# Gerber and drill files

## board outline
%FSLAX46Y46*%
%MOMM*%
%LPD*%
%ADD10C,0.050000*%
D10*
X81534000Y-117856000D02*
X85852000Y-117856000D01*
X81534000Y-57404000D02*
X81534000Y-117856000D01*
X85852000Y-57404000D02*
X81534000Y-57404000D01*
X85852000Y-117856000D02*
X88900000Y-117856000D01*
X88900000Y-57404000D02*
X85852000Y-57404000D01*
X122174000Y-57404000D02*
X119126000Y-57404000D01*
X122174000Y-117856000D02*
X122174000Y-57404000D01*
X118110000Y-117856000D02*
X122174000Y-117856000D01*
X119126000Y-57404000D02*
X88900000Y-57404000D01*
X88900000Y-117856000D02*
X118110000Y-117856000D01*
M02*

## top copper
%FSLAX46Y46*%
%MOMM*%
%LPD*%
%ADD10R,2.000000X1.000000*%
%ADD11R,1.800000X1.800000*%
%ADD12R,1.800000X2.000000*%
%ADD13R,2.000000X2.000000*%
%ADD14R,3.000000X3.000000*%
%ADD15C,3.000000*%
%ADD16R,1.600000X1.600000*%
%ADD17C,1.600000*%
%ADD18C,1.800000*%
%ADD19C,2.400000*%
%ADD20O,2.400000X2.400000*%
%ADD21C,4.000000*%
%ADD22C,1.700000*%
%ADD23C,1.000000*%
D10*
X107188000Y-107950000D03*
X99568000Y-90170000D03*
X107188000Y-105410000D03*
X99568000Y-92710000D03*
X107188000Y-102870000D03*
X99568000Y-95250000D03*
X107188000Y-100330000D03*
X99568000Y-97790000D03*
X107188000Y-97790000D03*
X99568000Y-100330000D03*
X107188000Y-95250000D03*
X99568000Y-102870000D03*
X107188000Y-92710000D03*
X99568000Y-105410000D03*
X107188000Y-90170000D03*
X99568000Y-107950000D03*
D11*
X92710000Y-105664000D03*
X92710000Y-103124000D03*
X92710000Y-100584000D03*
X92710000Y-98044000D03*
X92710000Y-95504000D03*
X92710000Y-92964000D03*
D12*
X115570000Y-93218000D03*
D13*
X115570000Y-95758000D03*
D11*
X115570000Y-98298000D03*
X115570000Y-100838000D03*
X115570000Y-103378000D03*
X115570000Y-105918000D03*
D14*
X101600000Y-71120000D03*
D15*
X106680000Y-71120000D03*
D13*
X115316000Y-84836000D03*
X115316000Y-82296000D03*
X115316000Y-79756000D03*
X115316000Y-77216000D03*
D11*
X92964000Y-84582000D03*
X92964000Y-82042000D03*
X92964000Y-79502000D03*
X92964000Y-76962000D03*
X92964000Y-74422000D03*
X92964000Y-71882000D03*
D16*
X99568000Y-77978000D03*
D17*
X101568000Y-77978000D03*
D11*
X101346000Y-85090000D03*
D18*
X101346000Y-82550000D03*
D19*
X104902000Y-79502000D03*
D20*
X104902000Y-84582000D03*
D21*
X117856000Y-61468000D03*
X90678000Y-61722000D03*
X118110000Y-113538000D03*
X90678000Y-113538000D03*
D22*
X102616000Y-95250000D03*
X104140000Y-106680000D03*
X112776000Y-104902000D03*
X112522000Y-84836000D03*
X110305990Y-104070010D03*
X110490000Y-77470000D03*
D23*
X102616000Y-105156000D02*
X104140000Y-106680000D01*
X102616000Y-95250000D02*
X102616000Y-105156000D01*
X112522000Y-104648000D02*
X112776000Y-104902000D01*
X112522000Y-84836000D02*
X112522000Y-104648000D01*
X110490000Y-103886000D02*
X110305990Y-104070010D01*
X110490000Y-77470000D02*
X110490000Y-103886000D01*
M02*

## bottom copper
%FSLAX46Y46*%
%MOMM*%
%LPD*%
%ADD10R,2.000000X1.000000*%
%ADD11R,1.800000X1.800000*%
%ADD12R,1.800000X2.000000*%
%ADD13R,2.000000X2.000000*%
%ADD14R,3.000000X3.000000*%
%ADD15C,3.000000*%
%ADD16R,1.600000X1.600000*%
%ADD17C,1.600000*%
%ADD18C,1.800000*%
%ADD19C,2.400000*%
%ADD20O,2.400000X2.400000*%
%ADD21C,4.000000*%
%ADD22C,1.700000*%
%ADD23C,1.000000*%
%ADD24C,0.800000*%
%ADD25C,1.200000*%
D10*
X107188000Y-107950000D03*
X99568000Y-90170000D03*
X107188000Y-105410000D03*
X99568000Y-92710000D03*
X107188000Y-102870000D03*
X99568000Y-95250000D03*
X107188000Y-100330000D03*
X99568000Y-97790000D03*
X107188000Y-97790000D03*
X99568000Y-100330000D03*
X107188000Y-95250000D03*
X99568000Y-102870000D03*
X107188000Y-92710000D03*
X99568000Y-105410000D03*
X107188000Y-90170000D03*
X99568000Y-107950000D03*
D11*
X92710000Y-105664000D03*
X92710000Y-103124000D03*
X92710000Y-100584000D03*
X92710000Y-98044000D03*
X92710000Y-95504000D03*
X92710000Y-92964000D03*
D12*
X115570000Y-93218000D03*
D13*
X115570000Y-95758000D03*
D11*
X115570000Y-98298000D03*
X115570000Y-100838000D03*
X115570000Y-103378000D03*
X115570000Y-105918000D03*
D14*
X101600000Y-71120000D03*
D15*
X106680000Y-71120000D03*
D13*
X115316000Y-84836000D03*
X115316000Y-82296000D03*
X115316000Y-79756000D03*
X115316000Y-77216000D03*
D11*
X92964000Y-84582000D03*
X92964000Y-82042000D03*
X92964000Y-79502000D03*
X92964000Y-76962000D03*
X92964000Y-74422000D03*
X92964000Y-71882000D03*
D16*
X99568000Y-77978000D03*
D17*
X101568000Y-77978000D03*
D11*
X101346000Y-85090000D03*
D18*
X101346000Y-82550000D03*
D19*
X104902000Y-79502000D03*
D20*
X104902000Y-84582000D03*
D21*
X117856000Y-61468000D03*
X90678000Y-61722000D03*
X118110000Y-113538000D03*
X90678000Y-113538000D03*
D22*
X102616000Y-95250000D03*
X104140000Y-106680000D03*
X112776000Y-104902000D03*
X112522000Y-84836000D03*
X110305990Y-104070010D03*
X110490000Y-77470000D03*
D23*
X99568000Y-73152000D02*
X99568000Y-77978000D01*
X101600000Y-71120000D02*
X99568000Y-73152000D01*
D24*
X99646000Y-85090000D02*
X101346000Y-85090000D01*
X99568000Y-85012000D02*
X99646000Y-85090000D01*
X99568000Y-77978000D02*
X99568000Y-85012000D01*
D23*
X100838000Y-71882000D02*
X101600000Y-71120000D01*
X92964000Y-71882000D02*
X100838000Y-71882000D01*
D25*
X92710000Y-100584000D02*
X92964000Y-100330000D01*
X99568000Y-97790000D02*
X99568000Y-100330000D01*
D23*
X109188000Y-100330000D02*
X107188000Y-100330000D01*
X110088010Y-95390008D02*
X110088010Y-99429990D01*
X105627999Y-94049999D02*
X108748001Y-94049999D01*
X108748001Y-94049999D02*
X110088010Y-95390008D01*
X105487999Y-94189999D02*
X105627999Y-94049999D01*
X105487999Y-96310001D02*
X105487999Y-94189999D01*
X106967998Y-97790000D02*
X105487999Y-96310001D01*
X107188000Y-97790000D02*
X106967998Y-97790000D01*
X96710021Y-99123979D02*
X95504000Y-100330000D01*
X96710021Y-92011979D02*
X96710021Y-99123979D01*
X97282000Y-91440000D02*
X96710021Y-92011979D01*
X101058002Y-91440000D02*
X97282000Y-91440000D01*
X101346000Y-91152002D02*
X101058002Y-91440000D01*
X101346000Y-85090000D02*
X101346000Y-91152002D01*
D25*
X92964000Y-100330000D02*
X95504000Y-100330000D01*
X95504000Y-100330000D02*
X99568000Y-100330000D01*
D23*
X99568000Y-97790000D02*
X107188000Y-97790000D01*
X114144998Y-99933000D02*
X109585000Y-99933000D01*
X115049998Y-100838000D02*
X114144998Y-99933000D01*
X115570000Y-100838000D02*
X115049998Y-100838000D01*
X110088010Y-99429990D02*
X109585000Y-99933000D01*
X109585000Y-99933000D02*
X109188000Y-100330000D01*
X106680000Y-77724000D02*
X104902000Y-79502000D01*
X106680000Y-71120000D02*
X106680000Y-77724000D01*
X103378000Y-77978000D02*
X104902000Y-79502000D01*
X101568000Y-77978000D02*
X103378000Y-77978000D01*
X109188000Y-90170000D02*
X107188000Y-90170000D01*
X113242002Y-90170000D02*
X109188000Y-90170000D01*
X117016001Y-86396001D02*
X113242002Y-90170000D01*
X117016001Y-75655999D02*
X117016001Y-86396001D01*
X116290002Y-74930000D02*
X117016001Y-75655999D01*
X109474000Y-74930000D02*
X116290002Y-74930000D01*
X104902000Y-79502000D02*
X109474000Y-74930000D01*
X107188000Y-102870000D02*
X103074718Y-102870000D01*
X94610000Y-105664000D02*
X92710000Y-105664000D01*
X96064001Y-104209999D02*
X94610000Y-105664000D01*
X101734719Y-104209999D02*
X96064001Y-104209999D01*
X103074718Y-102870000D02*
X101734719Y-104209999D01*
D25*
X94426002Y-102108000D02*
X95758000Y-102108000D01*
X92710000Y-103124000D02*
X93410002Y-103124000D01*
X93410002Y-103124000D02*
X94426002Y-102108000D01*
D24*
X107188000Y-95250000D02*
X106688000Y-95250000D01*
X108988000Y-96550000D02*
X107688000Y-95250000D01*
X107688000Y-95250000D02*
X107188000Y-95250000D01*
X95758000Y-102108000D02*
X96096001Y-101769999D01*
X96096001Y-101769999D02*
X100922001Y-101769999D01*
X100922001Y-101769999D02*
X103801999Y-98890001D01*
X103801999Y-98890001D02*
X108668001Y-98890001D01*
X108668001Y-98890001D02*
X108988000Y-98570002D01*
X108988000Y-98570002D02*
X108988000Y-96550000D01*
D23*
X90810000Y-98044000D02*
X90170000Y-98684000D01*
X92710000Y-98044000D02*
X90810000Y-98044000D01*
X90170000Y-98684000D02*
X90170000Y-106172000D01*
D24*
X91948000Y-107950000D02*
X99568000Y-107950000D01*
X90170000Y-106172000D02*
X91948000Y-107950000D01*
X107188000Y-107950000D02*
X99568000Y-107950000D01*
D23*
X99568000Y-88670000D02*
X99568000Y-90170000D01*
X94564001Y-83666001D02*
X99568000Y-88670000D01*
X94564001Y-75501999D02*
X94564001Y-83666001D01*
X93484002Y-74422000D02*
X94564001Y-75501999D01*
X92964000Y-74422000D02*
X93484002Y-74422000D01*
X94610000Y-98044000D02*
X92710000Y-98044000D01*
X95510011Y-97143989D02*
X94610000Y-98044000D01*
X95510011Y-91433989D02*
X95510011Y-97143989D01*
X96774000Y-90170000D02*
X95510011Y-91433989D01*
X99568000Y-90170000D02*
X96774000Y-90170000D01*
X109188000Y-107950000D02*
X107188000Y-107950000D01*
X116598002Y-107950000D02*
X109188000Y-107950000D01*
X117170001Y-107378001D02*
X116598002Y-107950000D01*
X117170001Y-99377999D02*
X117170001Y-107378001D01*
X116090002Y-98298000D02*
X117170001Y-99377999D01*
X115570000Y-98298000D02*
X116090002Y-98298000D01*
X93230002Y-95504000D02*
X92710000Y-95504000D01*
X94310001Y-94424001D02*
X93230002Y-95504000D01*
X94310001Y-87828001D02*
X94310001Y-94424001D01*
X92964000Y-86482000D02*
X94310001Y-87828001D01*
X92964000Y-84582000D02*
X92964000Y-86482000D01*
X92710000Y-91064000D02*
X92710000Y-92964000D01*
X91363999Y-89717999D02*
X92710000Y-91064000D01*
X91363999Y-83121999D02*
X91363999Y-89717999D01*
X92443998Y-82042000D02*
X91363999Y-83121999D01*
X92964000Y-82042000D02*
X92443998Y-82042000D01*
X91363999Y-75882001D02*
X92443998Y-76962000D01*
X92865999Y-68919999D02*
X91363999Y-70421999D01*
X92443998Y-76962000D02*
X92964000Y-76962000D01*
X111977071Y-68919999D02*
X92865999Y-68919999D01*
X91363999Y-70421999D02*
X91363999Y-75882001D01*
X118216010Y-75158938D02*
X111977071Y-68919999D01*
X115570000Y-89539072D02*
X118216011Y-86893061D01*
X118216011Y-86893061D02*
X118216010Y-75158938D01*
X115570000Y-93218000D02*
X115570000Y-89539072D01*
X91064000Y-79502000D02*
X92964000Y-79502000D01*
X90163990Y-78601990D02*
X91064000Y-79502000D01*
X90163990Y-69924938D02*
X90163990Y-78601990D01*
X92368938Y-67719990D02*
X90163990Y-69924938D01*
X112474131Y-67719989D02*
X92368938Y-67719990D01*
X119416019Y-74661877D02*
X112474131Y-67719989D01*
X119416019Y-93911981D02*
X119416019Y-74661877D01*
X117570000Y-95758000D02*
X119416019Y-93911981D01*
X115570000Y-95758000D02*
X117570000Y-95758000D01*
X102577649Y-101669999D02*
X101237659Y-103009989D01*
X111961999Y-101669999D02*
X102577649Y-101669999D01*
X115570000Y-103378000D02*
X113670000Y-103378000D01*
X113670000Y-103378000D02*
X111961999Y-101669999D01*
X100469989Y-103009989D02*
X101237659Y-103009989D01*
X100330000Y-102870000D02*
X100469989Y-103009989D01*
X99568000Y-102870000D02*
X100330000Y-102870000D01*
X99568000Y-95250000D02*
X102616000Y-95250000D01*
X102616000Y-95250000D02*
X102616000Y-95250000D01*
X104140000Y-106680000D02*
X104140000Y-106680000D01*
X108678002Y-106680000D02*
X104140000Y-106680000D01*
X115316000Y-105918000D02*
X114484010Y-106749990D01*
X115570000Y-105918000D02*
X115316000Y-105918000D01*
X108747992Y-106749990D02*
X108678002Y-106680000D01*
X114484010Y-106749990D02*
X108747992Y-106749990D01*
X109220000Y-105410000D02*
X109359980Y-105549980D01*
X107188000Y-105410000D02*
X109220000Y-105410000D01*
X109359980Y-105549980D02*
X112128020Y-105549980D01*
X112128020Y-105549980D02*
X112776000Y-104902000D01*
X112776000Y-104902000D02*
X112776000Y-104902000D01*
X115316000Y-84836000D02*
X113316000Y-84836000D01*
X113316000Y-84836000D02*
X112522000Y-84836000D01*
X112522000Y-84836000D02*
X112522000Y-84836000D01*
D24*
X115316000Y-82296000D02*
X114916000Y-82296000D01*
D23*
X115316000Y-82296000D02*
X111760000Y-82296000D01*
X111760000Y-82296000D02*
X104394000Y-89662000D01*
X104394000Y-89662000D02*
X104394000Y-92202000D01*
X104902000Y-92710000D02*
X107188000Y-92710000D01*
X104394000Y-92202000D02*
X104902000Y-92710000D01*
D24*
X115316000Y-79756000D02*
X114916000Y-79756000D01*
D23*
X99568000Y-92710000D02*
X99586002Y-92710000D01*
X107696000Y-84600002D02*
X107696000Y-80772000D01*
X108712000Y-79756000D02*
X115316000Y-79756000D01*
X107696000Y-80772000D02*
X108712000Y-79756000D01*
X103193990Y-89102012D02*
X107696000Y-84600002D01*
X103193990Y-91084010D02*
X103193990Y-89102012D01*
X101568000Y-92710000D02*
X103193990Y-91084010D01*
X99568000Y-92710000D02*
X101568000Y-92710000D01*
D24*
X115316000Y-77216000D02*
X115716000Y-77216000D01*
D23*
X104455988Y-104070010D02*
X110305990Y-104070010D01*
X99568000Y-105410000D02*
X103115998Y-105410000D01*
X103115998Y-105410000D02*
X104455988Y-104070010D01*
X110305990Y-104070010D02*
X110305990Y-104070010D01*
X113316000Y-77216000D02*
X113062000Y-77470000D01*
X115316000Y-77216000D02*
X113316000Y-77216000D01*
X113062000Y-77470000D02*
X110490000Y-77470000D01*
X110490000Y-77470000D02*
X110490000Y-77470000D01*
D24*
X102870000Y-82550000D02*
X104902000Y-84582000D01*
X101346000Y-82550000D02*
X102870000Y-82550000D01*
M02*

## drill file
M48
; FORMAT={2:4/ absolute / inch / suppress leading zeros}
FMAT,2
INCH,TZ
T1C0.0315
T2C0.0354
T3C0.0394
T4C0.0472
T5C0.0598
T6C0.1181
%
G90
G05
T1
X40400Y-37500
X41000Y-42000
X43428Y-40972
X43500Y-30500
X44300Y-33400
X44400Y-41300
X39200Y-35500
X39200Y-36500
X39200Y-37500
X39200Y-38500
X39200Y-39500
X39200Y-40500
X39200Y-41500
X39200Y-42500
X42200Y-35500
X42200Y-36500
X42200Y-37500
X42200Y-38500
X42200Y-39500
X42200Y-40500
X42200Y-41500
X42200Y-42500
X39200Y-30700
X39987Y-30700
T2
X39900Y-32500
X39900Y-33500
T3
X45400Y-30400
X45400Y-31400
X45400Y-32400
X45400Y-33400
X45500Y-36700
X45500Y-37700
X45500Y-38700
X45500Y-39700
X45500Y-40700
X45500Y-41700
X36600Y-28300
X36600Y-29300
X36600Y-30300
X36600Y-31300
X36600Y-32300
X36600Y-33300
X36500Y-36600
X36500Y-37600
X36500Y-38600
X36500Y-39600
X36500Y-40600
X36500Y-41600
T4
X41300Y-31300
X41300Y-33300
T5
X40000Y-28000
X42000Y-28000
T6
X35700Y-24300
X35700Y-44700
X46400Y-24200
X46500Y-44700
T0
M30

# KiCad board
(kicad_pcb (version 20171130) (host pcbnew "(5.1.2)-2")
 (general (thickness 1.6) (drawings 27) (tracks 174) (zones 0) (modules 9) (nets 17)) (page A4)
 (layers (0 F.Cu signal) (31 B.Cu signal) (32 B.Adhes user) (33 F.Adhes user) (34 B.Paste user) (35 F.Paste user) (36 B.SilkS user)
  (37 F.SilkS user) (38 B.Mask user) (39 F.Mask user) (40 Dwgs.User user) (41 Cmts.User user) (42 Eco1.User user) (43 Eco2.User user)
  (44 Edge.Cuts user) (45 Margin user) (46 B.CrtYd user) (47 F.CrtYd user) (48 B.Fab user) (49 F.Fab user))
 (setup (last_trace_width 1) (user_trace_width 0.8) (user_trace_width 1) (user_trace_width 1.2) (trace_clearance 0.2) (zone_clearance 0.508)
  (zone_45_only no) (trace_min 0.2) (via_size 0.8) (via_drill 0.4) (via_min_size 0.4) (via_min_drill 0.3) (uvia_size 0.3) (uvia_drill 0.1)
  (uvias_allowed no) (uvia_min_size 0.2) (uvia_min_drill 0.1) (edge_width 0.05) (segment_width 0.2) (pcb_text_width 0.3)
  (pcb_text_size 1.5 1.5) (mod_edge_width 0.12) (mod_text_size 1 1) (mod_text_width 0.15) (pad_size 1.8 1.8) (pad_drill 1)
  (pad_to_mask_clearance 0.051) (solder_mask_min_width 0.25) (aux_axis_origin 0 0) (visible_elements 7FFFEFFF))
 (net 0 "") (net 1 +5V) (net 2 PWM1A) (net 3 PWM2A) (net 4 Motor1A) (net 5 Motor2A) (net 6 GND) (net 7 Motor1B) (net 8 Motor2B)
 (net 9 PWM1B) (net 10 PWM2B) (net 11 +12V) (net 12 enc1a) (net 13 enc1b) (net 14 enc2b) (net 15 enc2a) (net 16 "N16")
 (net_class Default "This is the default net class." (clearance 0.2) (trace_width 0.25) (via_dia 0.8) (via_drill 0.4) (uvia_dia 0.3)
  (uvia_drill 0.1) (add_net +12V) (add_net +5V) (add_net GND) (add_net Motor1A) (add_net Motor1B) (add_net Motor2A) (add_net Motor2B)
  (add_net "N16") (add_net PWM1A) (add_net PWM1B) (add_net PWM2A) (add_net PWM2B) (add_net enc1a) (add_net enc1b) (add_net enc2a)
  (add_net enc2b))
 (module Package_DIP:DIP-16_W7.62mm (layer F.Cu) (at 107.188 107.95 180)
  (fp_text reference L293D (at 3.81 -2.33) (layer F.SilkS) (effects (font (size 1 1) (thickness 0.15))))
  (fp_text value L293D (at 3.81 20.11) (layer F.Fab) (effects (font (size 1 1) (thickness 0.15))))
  (pad 1 thru_hole rect (at 0 0 180) (size 2 1) (drill 0.8) (layers *.Cu *.Mask) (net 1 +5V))
  (pad 9 thru_hole rect (at 7.62 17.78 180) (size 2 1) (drill 0.8) (layers *.Cu *.Mask) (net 1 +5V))
  (pad 2 thru_hole rect (at 0 2.54 180) (size 2 1) (drill 0.8) (layers *.Cu *.Mask) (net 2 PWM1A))
  (pad 10 thru_hole rect (at 7.62 15.24 180) (size 2 1) (drill 0.8) (layers *.Cu *.Mask) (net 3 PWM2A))
  (pad 3 thru_hole rect (at 0 5.08 180) (size 2 1) (drill 0.8) (layers *.Cu *.Mask) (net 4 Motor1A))
  (pad 11 thru_hole rect (at 7.62 12.7 180) (size 2 1) (drill 0.8) (layers *.Cu *.Mask) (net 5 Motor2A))
  (pad 4 thru_hole rect (at 0 7.62 180) (size 2 1) (drill 0.8) (layers *.Cu *.Mask) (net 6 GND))
  (pad 12 thru_hole rect (at 7.62 10.16 180) (size 2 1) (drill 0.8) (layers *.Cu *.Mask) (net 6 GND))
  (pad 5 thru_hole rect (at 0 10.16 180) (size 2 1) (drill 0.8) (layers *.Cu *.Mask) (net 6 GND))
  (pad 13 thru_hole rect (at 7.62 7.62 180) (size 2 1) (drill 0.8) (layers *.Cu *.Mask) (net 6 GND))
  (pad 6 thru_hole rect (at 0 12.7 180) (size 2 1) (drill 0.8) (layers *.Cu *.Mask) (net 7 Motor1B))
  (pad 14 thru_hole rect (at 7.62 5.08 180) (size 2 1) (drill 0.8) (layers *.Cu *.Mask) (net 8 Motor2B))
  (pad 7 thru_hole rect (at 0 15.24 180) (size 2 1) (drill 0.8) (layers *.Cu *.Mask) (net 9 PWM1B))
  (pad 15 thru_hole rect (at 7.62 2.54 180) (size 2 1) (drill 0.8) (layers *.Cu *.Mask) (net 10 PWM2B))
  (pad 8 thru_hole rect (at 0 17.78 180) (size 2 1) (drill 0.8) (layers *.Cu *.Mask) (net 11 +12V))
  (pad 16 thru_hole rect (at 7.62 0 180) (size 2 1) (drill 0.8) (layers *.Cu *.Mask) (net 1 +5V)))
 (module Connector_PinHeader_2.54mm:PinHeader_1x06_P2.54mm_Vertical (layer F.Cu) (at 92.71 105.664 180)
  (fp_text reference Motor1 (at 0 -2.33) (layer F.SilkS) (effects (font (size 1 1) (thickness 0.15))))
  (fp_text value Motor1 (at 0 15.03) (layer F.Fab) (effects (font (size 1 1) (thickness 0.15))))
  (pad 1 thru_hole rect (at 0 0 180) (size 1.8 1.8) (drill 1) (layers *.Cu *.Mask) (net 4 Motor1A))
  (pad 2 thru_hole rect (at 0 2.54 180) (size 1.8 1.8) (drill 1) (layers *.Cu *.Mask) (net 7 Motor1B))
  (pad 3 thru_hole rect (at 0 5.08 180) (size 1.8 1.8) (drill 1) (layers *.Cu *.Mask) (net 6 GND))
  (pad 4 thru_hole rect (at 0 7.62 180) (size 1.8 1.8) (drill 1) (layers *.Cu *.Mask) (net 1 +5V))
  (pad 5 thru_hole rect (at 0 10.16 180) (size 1.8 1.8) (drill 1) (layers *.Cu *.Mask) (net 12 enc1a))
  (pad 6 thru_hole rect (at 0 12.7 180) (size 1.8 1.8) (drill 1) (layers *.Cu *.Mask) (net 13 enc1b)))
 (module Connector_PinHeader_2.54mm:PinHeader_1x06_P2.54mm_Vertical (layer F.Cu) (at 115.57 105.918 180)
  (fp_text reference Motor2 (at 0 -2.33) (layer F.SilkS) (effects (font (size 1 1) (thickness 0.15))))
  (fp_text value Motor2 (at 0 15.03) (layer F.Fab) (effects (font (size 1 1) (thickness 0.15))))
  (pad 6 thru_hole rect (at 0 12.7 180) (size 1.8 2) (drill 1) (layers *.Cu *.Mask) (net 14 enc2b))
  (pad 5 thru_hole rect (at 0 10.16 180) (size 2 2) (drill 1) (layers *.Cu *.Mask) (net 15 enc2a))
  (pad 4 thru_hole rect (at 0 7.62 180) (size 1.8 1.8) (drill 1) (layers *.Cu *.Mask) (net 1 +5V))
  (pad 3 thru_hole rect (at 0 5.08 180) (size 1.8 1.8) (drill 1) (layers *.Cu *.Mask) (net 6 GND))
  (pad 2 thru_hole rect (at 0 2.54 180) (size 1.8 1.8) (drill 1) (layers *.Cu *.Mask) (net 8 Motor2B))
  (pad 1 thru_hole rect (at 0 0 180) (size 1.8 1.8) (drill 1) (layers *.Cu *.Mask) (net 5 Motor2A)))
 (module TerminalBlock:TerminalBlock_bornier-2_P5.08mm (layer F.Cu) (at 101.6 71.12)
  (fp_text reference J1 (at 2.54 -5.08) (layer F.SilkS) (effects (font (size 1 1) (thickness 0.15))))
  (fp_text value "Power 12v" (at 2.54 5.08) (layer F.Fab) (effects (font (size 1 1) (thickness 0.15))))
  (pad 1 thru_hole rect (at 0 0) (size 3 3) (drill 1.52) (layers *.Cu *.Mask) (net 6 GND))
  (pad 2 thru_hole circle (at 5.08 0) (size 3 3) (drill 1.52) (layers *.Cu *.Mask) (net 11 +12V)))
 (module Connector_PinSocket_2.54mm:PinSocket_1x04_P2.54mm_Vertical (layer F.Cu) (at 115.316 84.836 180)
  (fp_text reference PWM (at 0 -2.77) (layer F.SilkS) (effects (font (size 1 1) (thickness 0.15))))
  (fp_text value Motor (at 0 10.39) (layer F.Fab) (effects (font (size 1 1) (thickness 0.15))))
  (pad 1 thru_hole rect (at 0 0 180) (size 2 2) (drill 1) (layers *.Cu *.Mask) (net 2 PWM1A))
  (pad 2 thru_hole rect (at 0 2.54 180) (size 2 2) (drill 1) (layers *.Cu *.Mask) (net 9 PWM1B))
  (pad 3 thru_hole rect (at 0 5.08 180) (size 2 2) (drill 1) (layers *.Cu *.Mask) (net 3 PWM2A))
  (pad 4 thru_hole rect (at 0 7.62 180) (size 2 2) (drill 1) (layers *.Cu *.Mask) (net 10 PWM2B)))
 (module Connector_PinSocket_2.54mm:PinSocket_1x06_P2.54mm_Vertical (layer F.Cu) (at 92.964 84.582 180)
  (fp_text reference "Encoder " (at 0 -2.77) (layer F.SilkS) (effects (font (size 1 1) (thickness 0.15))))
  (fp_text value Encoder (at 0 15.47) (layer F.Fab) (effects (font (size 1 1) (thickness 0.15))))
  (pad 1 thru_hole rect (at 0 0 180) (size 1.8 1.8) (drill 1) (layers *.Cu *.Mask) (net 12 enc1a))
  (pad 2 thru_hole rect (at 0 2.54 180) (size 1.8 1.8) (drill 1) (layers *.Cu *.Mask) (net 13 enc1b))
  (pad 3 thru_hole rect (at 0 5.08 180) (size 1.8 1.8) (drill 1) (layers *.Cu *.Mask) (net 15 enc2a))
  (pad 4 thru_hole rect (at 0 7.62 180) (size 1.8 1.8) (drill 1) (layers *.Cu *.Mask) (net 14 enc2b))
  (pad 5 thru_hole rect (at 0 10.16 180) (size 1.8 1.8) (drill 1) (layers *.Cu *.Mask) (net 1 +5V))
  (pad 6 thru_hole rect (at 0 12.7 180) (size 1.8 1.8) (drill 1) (layers *.Cu *.Mask) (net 6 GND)))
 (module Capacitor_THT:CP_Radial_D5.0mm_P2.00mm (layer F.Cu) (at 99.568 77.978)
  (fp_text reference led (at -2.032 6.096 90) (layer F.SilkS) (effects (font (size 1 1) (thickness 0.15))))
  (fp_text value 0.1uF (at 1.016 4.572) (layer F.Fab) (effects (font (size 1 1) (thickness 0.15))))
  (pad 1 thru_hole rect (at 0 0) (size 1.6 1.6) (drill 0.8) (layers *.Cu *.Mask) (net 6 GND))
  (pad 2 thru_hole circle (at 2 0) (size 1.6 1.6) (drill 0.8) (layers *.Cu *.Mask) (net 11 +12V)))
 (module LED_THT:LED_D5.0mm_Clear (layer F.Cu) (at 101.346 85.09 90)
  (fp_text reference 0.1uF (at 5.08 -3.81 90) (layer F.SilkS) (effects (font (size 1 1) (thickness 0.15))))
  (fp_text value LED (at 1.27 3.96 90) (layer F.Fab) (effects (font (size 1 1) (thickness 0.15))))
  (pad 1 thru_hole rect (at 0 0 90) (size 1.8 1.8) (drill 0.9) (layers *.Cu *.Mask) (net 6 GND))
  (pad 2 thru_hole circle (at 2.54 0 90) (size 1.8 1.8) (drill 0.9) (layers *.Cu *.Mask) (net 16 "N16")))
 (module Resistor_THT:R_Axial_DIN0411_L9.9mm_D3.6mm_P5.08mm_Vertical (layer F.Cu) (at 104.902 79.502 270)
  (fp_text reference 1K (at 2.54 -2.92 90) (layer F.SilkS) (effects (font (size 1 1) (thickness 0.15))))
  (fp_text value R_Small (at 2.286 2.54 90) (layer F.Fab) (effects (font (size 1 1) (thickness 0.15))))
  (pad 1 thru_hole circle (at 0 0 270) (size 2.4 2.4) (drill 1.2) (layers *.Cu *.Mask) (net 11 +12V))
  (pad 2 thru_hole oval (at 5.08 0 270) (size 2.4 2.4) (drill 1.2) (layers *.Cu *.Mask) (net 16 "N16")))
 (gr_line (start 81.534 117.856) (end 85.852 117.856) (layer Edge.Cuts) (width 0.05))
 (gr_line (start 81.534 57.404) (end 81.534 117.856) (layer Edge.Cuts) (width 0.05))
 (gr_line (start 85.852 57.404) (end 81.534 57.404) (layer Edge.Cuts) (width 0.05))
 (gr_line (start 85.852 117.856) (end 88.9 117.856) (layer Edge.Cuts) (width 0.05))
 (gr_line (start 88.9 57.404) (end 85.852 57.404) (layer Edge.Cuts) (width 0.05))
 (gr_line (start 122.174 57.404) (end 119.126 57.404) (layer Edge.Cuts) (width 0.05))
 (gr_line (start 122.174 117.856) (end 122.174 57.404) (layer Edge.Cuts) (width 0.05))
 (gr_line (start 118.11 117.856) (end 122.174 117.856) (layer Edge.Cuts) (width 0.05))
 (gr_line (start 119.126 57.404) (end 88.9 57.404) (layer Edge.Cuts) (width 0.05))
 (gr_line (start 88.9 117.856) (end 118.11 117.856) (layer Edge.Cuts) (width 0.05))
 (via (at 117.856 61.468) (size 4) (drill 3) (layers F.Cu B.Cu) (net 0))
 (via (at 90.678 61.722) (size 4) (drill 3) (layers F.Cu B.Cu) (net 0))
 (via (at 118.11 113.538) (size 4) (drill 3) (layers F.Cu B.Cu) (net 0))
 (via (at 90.678 113.538) (size 4) (drill 3) (layers F.Cu B.Cu) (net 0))
 (segment (start 99.568 73.152) (end 99.568 77.978) (width 1) (layer B.Cu) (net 6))
 (segment (start 101.6 71.12) (end 99.568 73.152) (width 1) (layer B.Cu) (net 6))
 (segment (start 99.646 85.09) (end 101.346 85.09) (width 0.8) (layer B.Cu) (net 6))
 (segment (start 99.568 85.012) (end 99.646 85.09) (width 0.8) (layer B.Cu) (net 6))
 (segment (start 99.568 77.978) (end 99.568 85.012) (width 0.8) (layer B.Cu) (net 6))
 (segment (start 100.838 71.882) (end 101.6 71.12) (width 1) (layer B.Cu) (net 6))
 (segment (start 92.964 71.882) (end 100.838 71.882) (width 1) (layer B.Cu) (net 6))
 (segment (start 92.71 100.584) (end 92.964 100.33) (width 1.2) (layer B.Cu) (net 6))
 (segment (start 99.568 97.79) (end 99.568 100.33) (width 1.2) (layer B.Cu) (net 6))
 (segment (start 109.188 100.33) (end 107.188 100.33) (width 1) (layer B.Cu) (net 6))
 (segment (start 110.08801 95.390008) (end 110.08801 99.42999) (width 1) (layer B.Cu) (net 6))
 (segment (start 105.627999 94.049999) (end 108.748001 94.049999) (width 1) (layer B.Cu) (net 6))
 (segment (start 108.748001 94.049999) (end 110.08801 95.390008) (width 1) (layer B.Cu) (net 6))
 (segment (start 105.487999 94.189999) (end 105.627999 94.049999) (width 1) (layer B.Cu) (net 6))
 (segment (start 105.487999 96.310001) (end 105.487999 94.189999) (width 1) (layer B.Cu) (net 6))
 (segment (start 106.967998 97.79) (end 105.487999 96.310001) (width 1) (layer B.Cu) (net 6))
 (segment (start 107.188 97.79) (end 106.967998 97.79) (width 1) (layer B.Cu) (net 6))
 (segment (start 96.710021 99.123979) (end 95.504 100.33) (width 1) (layer B.Cu) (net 6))
 (segment (start 96.710021 92.011979) (end 96.710021 99.123979) (width 1) (layer B.Cu) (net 6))
 (segment (start 97.282 91.44) (end 96.710021 92.011979) (width 1) (layer B.Cu) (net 6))
 (segment (start 101.058002 91.44) (end 97.282 91.44) (width 1) (layer B.Cu) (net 6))
 (segment (start 101.346 91.152002) (end 101.058002 91.44) (width 1) (layer B.Cu) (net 6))
 (segment (start 101.346 85.09) (end 101.346 91.152002) (width 1) (layer B.Cu) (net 6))
 (segment (start 92.964 100.33) (end 95.504 100.33) (width 1.2) (layer B.Cu) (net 6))
 (segment (start 95.504 100.33) (end 99.568 100.33) (width 1.2) (layer B.Cu) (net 6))
 (segment (start 99.568 97.79) (end 107.188 97.79) (width 1) (layer B.Cu) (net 6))
 (segment (start 114.144998 99.933) (end 109.585 99.933) (width 1) (layer B.Cu) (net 6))
 (segment (start 115.049998 100.838) (end 114.144998 99.933) (width 1) (layer B.Cu) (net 6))
 (segment (start 115.57 100.838) (end 115.049998 100.838) (width 1) (layer B.Cu) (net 6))
 (segment (start 110.08801 99.42999) (end 109.585 99.933) (width 1) (layer B.Cu) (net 6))
 (segment (start 109.585 99.933) (end 109.188 100.33) (width 1) (layer B.Cu) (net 6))
 (segment (start 106.68 77.724) (end 104.902 79.502) (width 1) (layer B.Cu) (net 11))
 (segment (start 106.68 71.12) (end 106.68 77.724) (width 1) (layer B.Cu) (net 11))
 (segment (start 103.378 77.978) (end 104.902 79.502) (width 1) (layer B.Cu) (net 11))
 (segment (start 101.568 77.978) (end 103.378 77.978) (width 1) (layer B.Cu) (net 11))
 (segment (start 109.188 90.17) (end 107.188 90.17) (width 1) (layer B.Cu) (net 11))
 (segment (start 113.242002 90.17) (end 109.188 90.17) (width 1) (layer B.Cu) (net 11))
 (segment (start 117.016001 86.396001) (end 113.242002 90.17) (width 1) (layer B.Cu) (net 11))
 (segment (start 117.016001 75.655999) (end 117.016001 86.396001) (width 1) (layer B.Cu) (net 11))
 (segment (start 116.290002 74.93) (end 117.016001 75.655999) (width 1) (layer B.Cu) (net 11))
 (segment (start 109.474 74.93) (end 116.290002 74.93) (width 1) (layer B.Cu) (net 11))
 (segment (start 104.902 79.502) (end 109.474 74.93) (width 1) (layer B.Cu) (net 11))
 (segment (start 107.188 102.87) (end 103.074718 102.87) (width 1) (layer B.Cu) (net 4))
 (segment (start 94.61 105.664) (end 92.71 105.664) (width 1) (layer B.Cu) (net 4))
 (segment (start 96.064001 104.209999) (end 94.61 105.664) (width 1) (layer B.Cu) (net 4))
 (segment (start 101.734719 104.209999) (end 96.064001 104.209999) (width 1) (layer B.Cu) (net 4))
 (segment (start 103.074718 102.87) (end 101.734719 104.209999) (width 1) (layer B.Cu) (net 4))
 (segment (start 94.426002 102.108) (end 95.758 102.108) (width 1.2) (layer B.Cu) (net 7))
 (segment (start 92.71 103.124) (end 93.410002 103.124) (width 1.2) (layer B.Cu) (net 7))
 (segment (start 93.410002 103.124) (end 94.426002 102.108) (width 1.2) (layer B.Cu) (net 7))
 (segment (start 107.188 95.25) (end 106.688 95.25) (width 0.8) (layer B.Cu) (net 7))
 (segment (start 108.988 96.55) (end 107.688 95.25) (width 0.8) (layer B.Cu) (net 7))
 (segment (start 107.688 95.25) (end 107.188 95.25) (width 0.8) (layer B.Cu) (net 7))
 (segment (start 95.758 102.108) (end 96.096001 101.769999) (width 0.8) (layer B.Cu) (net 7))
 (segment (start 96.096001 101.769999) (end 100.922001 101.769999) (width 0.8) (layer B.Cu) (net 7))
 (segment (start 100.922001 101.769999) (end 103.801999 98.890001) (width 0.8) (layer B.Cu) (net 7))
 (segment (start 103.801999 98.890001) (end 108.668001 98.890001) (width 0.8) (layer B.Cu) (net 7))
 (segment (start 108.668001 98.890001) (end 108.988 98.570002) (width 0.8) (layer B.Cu) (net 7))
 (segment (start 108.988 98.570002) (end 108.988 96.55) (width 0.8) (layer B.Cu) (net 7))
 (segment (start 90.81 98.044) (end 90.17 98.684) (width 1) (layer B.Cu) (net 1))
 (segment (start 92.71 98.044) (end 90.81 98.044) (width 1) (layer B.Cu) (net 1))
 (segment (start 90.17 98.684) (end 90.17 106.172) (width 1) (layer B.Cu) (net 1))
 (segment (start 91.948 107.95) (end 99.568 107.95) (width 0.8) (layer B.Cu) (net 1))
 (segment (start 90.17 106.172) (end 91.948 107.95) (width 0.8) (layer B.Cu) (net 1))
 (segment (start 107.188 107.95) (end 99.568 107.95) (width 0.8) (layer B.Cu) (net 1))
 (segment (start 99.568 88.67) (end 99.568 90.17) (width 1) (layer B.Cu) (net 1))
 (segment (start 94.564001 83.666001) (end 99.568 88.67) (width 1) (layer B.Cu) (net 1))
 (segment (start 94.564001 75.501999) (end 94.564001 83.666001) (width 1) (layer B.Cu) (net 1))
 (segment (start 93.484002 74.422) (end 94.564001 75.501999) (width 1) (layer B.Cu) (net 1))
 (segment (start 92.964 74.422) (end 93.484002 74.422) (width 1) (layer B.Cu) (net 1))
 (segment (start 94.61 98.044) (end 92.71 98.044) (width 1) (layer B.Cu) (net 1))
 (segment (start 95.510011 97.143989) (end 94.61 98.044) (width 1) (layer B.Cu) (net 1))
 (segment (start 95.510011 91.433989) (end 95.510011 97.143989) (width 1) (layer B.Cu) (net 1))
 (segment (start 96.774 90.17) (end 95.510011 91.433989) (width 1) (layer B.Cu) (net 1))
 (segment (start 99.568 90.17) (end 96.774 90.17) (width 1) (layer B.Cu) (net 1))
 (segment (start 109.188 107.95) (end 107.188 107.95) (width 1) (layer B.Cu) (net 1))
 (segment (start 116.598002 107.95) (end 109.188 107.95) (width 1) (layer B.Cu) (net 1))
 (segment (start 117.170001 107.378001) (end 116.598002 107.95) (width 1) (layer B.Cu) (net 1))
 (segment (start 117.170001 99.377999) (end 117.170001 107.378001) (width 1) (layer B.Cu) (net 1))
 (segment (start 116.090002 98.298) (end 117.170001 99.377999) (width 1) (layer B.Cu) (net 1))
 (segment (start 115.57 98.298) (end 116.090002 98.298) (width 1) (layer B.Cu) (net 1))
 (segment (start 93.230002 95.504) (end 92.71 95.504) (width 1) (layer B.Cu) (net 12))
 (segment (start 94.310001 94.424001) (end 93.230002 95.504) (width 1) (layer B.Cu) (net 12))
 (segment (start 94.310001 87.828001) (end 94.310001 94.424001) (width 1) (layer B.Cu) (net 12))
 (segment (start 92.964 86.482) (end 94.310001 87.828001) (width 1) (layer B.Cu) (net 12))
 (segment (start 92.964 84.582) (end 92.964 86.482) (width 1) (layer B.Cu) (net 12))
 (segment (start 92.71 91.064) (end 92.71 92.964) (width 1) (layer B.Cu) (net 13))
 (segment (start 91.363999 89.717999) (end 92.71 91.064) (width 1) (layer B.Cu) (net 13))
 (segment (start 91.363999 83.121999) (end 91.363999 89.717999) (width 1) (layer B.Cu) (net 13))
 (segment (start 92.443998 82.042) (end 91.363999 83.121999) (width 1) (layer B.Cu) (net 13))
 (segment (start 92.964 82.042) (end 92.443998 82.042) (width 1) (layer B.Cu) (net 13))
 (segment (start 91.363999 75.882001) (end 92.443998 76.962) (width 1) (layer B.Cu) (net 14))
 (segment (start 92.865999 68.919999) (end 91.363999 70.421999) (width 1) (layer B.Cu) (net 14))
 (segment (start 92.443998 76.962) (end 92.964 76.962) (width 1) (layer B.Cu) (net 14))
 (segment (start 111.977071 68.919999) (end 92.865999 68.919999) (width 1) (layer B.Cu) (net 14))
 (segment (start 91.363999 70.421999) (end 91.363999 75.882001) (width 1) (layer B.Cu) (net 14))
 (segment (start 118.21601 75.158938) (end 111.977071 68.919999) (width 1) (layer B.Cu) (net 14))
 (segment (start 115.57 89.539072) (end 118.216011 86.893061) (width 1) (layer B.Cu) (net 14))
 (segment (start 118.216011 86.893061) (end 118.21601 75.158938) (width 1) (layer B.Cu) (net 14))
 (segment (start 115.57 93.218) (end 115.57 89.539072) (width 1) (layer B.Cu) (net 14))
 (segment (start 91.064 79.502) (end 92.964 79.502) (width 1) (layer B.Cu) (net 15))
 (segment (start 90.16399 78.60199) (end 91.064 79.502) (width 1) (layer B.Cu) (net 15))
 (segment (start 90.16399 69.924938) (end 90.16399 78.60199) (width 1) (layer B.Cu) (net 15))
 (segment (start 92.368938 67.71999) (end 90.16399 69.924938) (width 1) (layer B.Cu) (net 15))
 (segment (start 112.474131 67.719989) (end 92.368938 67.71999) (width 1) (layer B.Cu) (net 15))
 (segment (start 119.416019 74.661877) (end 112.474131 67.719989) (width 1) (layer B.Cu) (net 15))
 (segment (start 119.416019 93.911981) (end 119.416019 74.661877) (width 1) (layer B.Cu) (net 15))
 (segment (start 117.57 95.758) (end 119.416019 93.911981) (width 1) (layer B.Cu) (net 15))
 (segment (start 115.57 95.758) (end 117.57 95.758) (width 1) (layer B.Cu) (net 15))
 (segment (start 102.577649 101.669999) (end 101.237659 103.009989) (width 1) (layer B.Cu) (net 8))
 (segment (start 111.961999 101.669999) (end 102.577649 101.669999) (width 1) (layer B.Cu) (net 8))
 (segment (start 115.57 103.378) (end 113.67 103.378) (width 1) (layer B.Cu) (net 8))
 (segment (start 113.67 103.378) (end 111.961999 101.669999) (width 1) (layer B.Cu) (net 8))
 (segment (start 100.469989 103.009989) (end 101.237659 103.009989) (width 1) (layer B.Cu) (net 8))
 (segment (start 100.33 102.87) (end 100.469989 103.009989) (width 1) (layer B.Cu) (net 8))
 (segment (start 99.568 102.87) (end 100.33 102.87) (width 1) (layer B.Cu) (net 8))
 (segment (start 99.568 95.25) (end 102.616 95.25) (width 1) (layer B.Cu) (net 5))
 (segment (start 102.616 95.25) (end 102.616 95.25) (width 1) (layer B.Cu) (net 5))
 (via (at 102.616 95.25) (size 1.7) (drill 0.8) (layers F.Cu B.Cu) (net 5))
 (segment (start 104.14 106.68) (end 104.14 106.68) (width 1) (layer B.Cu) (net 5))
 (via (at 104.14 106.68) (size 1.7) (drill 0.8) (layers F.Cu B.Cu) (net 5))
 (segment (start 108.678002 106.68) (end 104.14 106.68) (width 1) (layer B.Cu) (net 5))
 (segment (start 115.316 105.918) (end 114.48401 106.74999) (width 1) (layer B.Cu) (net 5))
 (segment (start 115.57 105.918) (end 115.316 105.918) (width 1) (layer B.Cu) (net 5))
 (segment (start 108.747992 106.74999) (end 108.678002 106.68) (width 1) (layer B.Cu) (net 5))
 (segment (start 114.48401 106.74999) (end 108.747992 106.74999) (width 1) (layer B.Cu) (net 5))
 (segment (start 102.616 105.156) (end 104.14 106.68) (width 1) (layer F.Cu) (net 5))
 (segment (start 102.616 95.25) (end 102.616 105.156) (width 1) (layer F.Cu) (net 5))
 (segment (start 109.22 105.41) (end 109.35998 105.54998) (width 1) (layer B.Cu) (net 2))
 (segment (start 107.188 105.41) (end 109.22 105.41) (width 1) (layer B.Cu) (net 2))
 (segment (start 109.35998 105.54998) (end 112.12802 105.54998) (width 1) (layer B.Cu) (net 2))
 (segment (start 112.12802 105.54998) (end 112.776 104.902) (width 1) (layer B.Cu) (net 2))
 (segment (start 112.776 104.902) (end 112.776 104.902) (width 1) (layer B.Cu) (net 2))
 (via (at 112.776 104.902) (size 1.7) (drill 0.8) (layers F.Cu B.Cu) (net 2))
 (segment (start 115.316 84.836) (end 113.316 84.836) (width 1) (layer B.Cu) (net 2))
 (segment (start 113.316 84.836) (end 112.522 84.836) (width 1) (layer B.Cu) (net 2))
 (segment (start 112.522 84.836) (end 112.522 84.836) (width 1) (layer B.Cu) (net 2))
 (via (at 112.522 84.836) (size 1.7) (drill 0.8) (layers F.Cu B.Cu) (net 2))
 (segment (start 112.522 104.648) (end 112.776 104.902) (width 1) (layer F.Cu) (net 2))
 (segment (start 112.522 84.836) (end 112.522 104.648) (width 1) (layer F.Cu) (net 2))
 (segment (start 115.316 82.296) (end 114.916 82.296) (width 0.8) (layer B.Cu) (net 9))
 (segment (start 115.316 82.296) (end 111.76 82.296) (width 1) (layer B.Cu) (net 9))
 (segment (start 111.76 82.296) (end 104.394 89.662) (width 1) (layer B.Cu) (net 9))
 (segment (start 104.394 89.662) (end 104.394 92.202) (width 1) (layer B.Cu) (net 9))
 (segment (start 104.902 92.71) (end 107.188 92.71) (width 1) (layer B.Cu) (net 9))
 (segment (start 104.394 92.202) (end 104.902 92.71) (width 1) (layer B.Cu) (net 9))
 (segment (start 115.316 79.756) (end 114.916 79.756) (width 0.8) (layer B.Cu) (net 3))
 (segment (start 99.568 92.71) (end 99.586002 92.71) (width 1) (layer B.Cu) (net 3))
 (segment (start 107.696 84.600002) (end 107.696 80.772) (width 1) (layer B.Cu) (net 3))
 (segment (start 108.712 79.756) (end 115.316 79.756) (width 1) (layer B.Cu) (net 3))
 (segment (start 107.696 80.772) (end 108.712 79.756) (width 1) (layer B.Cu) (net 3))
 (segment (start 103.19399 89.102012) (end 107.696 84.600002) (width 1) (layer B.Cu) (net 3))
 (segment (start 103.19399 91.08401) (end 103.19399 89.102012) (width 1) (layer B.Cu) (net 3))
 (segment (start 101.568 92.71) (end 103.19399 91.08401) (width 1) (layer B.Cu) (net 3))
 (segment (start 99.568 92.71) (end 101.568 92.71) (width 1) (layer B.Cu) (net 3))
 (segment (start 115.316 77.216) (end 115.716 77.216) (width 0.8) (layer B.Cu) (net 10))
 (segment (start 104.455988 104.07001) (end 110.30599 104.07001) (width 1) (layer B.Cu) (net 10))
 (segment (start 99.568 105.41) (end 103.115998 105.41) (width 1) (layer B.Cu) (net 10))
 (segment (start 103.115998 105.41) (end 104.455988 104.07001) (width 1) (layer B.Cu) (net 10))
 (segment (start 110.30599 104.07001) (end 110.30599 104.07001) (width 1) (layer B.Cu) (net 10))
 (via (at 110.30599 104.07001) (size 1.7) (drill 0.8) (layers F.Cu B.Cu) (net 10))
 (segment (start 113.316 77.216) (end 113.062 77.47) (width 1) (layer B.Cu) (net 10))
 (segment (start 115.316 77.216) (end 113.316 77.216) (width 1) (layer B.Cu) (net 10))
 (segment (start 113.062 77.47) (end 110.49 77.47) (width 1) (layer B.Cu) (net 10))
 (segment (start 110.49 77.47) (end 110.49 77.47) (width 1) (layer B.Cu) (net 10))
 (via (at 110.49 77.47) (size 1.7) (drill 0.8) (layers F.Cu B.Cu) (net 10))
 (segment (start 110.49 103.886) (end 110.30599 104.07001) (width 1) (layer F.Cu) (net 10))
 (segment (start 110.49 77.47) (end 110.49 103.886) (width 1) (layer F.Cu) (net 10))
 (segment (start 102.87 82.55) (end 104.902 84.582) (width 0.8) (layer B.Cu) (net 16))
 (segment (start 101.346 82.55) (end 102.87 82.55) (width 0.8) (layer B.Cu) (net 16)))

